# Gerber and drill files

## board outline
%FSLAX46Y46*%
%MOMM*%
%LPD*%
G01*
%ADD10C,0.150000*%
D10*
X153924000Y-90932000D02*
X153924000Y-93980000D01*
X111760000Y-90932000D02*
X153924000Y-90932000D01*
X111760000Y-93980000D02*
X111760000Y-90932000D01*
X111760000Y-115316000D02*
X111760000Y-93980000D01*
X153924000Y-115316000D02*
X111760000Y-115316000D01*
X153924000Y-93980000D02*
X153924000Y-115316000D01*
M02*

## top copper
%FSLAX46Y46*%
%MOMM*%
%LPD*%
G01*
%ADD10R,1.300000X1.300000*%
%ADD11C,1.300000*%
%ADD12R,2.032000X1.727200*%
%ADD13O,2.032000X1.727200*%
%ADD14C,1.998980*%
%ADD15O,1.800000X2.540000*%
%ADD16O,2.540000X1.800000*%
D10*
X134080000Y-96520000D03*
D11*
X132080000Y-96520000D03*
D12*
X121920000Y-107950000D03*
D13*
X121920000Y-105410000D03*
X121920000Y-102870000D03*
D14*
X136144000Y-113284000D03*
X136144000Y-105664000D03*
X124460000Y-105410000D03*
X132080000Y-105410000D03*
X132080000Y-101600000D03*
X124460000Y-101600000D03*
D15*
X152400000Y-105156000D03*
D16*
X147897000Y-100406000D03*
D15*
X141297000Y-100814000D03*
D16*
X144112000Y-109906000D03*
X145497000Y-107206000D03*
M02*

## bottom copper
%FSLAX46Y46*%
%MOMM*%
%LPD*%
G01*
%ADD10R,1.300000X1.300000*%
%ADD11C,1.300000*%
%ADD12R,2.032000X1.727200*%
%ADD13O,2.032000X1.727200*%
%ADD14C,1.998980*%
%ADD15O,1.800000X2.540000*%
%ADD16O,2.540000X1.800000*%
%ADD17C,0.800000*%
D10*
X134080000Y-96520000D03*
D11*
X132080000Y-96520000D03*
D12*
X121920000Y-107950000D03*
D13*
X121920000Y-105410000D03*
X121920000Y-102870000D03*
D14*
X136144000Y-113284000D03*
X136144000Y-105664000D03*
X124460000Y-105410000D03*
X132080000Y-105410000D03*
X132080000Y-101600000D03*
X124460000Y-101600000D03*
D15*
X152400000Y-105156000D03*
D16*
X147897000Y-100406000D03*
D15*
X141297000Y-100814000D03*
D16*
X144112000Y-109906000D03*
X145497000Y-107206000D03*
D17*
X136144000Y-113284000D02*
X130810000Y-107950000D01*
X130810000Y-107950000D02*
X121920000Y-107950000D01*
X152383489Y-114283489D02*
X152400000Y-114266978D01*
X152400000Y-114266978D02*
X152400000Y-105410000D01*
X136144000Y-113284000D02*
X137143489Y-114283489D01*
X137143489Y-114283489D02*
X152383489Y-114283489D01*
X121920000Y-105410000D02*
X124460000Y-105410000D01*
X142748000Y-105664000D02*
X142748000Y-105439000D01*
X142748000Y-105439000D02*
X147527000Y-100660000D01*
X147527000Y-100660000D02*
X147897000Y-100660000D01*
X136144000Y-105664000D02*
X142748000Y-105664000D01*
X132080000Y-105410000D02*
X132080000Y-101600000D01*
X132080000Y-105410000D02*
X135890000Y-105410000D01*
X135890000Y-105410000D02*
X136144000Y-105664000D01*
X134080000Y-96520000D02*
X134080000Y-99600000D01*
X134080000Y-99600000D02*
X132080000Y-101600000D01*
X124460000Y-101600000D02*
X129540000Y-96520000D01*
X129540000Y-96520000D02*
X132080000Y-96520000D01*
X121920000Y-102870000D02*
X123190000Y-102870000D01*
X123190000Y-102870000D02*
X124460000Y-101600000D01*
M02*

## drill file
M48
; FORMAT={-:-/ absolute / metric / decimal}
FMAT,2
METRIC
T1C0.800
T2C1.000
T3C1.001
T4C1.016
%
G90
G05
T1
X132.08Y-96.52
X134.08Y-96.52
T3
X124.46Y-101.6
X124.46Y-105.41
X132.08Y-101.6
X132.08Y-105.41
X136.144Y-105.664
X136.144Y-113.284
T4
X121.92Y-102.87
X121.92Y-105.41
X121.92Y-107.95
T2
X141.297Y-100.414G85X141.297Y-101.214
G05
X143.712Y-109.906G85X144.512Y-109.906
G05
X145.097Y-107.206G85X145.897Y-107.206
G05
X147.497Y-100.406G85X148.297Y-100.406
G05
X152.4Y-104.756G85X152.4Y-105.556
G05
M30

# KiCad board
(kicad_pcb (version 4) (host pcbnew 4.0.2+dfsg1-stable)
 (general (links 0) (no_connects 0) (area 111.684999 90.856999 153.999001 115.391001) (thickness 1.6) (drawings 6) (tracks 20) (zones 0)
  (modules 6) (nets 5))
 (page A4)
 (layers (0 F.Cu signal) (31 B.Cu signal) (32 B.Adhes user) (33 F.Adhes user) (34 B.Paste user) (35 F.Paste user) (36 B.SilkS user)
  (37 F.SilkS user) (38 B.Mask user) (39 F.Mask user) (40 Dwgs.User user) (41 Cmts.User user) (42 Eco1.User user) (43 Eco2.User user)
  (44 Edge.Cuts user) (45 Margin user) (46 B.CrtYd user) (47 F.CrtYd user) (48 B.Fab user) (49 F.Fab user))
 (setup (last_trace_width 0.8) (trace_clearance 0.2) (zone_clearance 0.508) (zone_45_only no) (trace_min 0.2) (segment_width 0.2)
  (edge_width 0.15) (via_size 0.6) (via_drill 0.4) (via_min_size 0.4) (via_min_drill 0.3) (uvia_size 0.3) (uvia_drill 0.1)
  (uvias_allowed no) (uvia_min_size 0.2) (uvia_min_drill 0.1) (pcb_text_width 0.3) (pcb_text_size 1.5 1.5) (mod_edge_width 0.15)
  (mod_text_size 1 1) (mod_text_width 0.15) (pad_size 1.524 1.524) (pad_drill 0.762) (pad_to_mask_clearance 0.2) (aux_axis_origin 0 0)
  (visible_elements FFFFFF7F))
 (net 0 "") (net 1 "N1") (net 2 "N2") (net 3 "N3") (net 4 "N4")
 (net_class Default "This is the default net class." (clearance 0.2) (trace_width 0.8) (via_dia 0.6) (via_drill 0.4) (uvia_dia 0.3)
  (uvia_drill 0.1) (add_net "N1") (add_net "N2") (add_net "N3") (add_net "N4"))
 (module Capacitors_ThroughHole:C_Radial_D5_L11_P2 (layer F.Cu) (at 134.08 96.52 180)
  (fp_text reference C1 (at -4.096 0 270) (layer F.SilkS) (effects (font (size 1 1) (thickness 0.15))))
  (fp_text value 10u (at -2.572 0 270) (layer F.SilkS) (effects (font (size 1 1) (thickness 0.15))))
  (pad 1 thru_hole rect (at 0 0 180) (size 1.3 1.3) (drill 0.8) (layers *.Cu *.Mask F.SilkS) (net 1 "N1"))
  (pad 2 thru_hole circle (at 2 0 180) (size 1.3 1.3) (drill 0.8) (layers *.Cu *.Mask F.SilkS) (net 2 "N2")))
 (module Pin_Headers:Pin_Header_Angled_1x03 (layer F.Cu) (at 121.92 107.95 180)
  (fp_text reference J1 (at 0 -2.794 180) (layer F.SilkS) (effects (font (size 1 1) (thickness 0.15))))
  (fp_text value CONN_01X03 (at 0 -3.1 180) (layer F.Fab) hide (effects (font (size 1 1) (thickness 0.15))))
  (pad 1 thru_hole rect (at 0 0 180) (size 2.032 1.7272) (drill 1.016) (layers *.Cu *.Mask F.SilkS) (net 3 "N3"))
  (pad 2 thru_hole oval (at 0 2.54 180) (size 2.032 1.7272) (drill 1.016) (layers *.Cu *.Mask F.SilkS) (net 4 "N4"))
  (pad 3 thru_hole oval (at 0 5.08 180) (size 2.032 1.7272) (drill 1.016) (layers *.Cu *.Mask F.SilkS) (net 2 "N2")))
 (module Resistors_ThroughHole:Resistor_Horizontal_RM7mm (layer F.Cu) (at 136.144 113.284 90)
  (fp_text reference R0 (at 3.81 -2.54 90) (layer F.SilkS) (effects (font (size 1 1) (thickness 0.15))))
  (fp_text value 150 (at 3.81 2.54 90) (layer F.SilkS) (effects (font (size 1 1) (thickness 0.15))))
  (pad 1 thru_hole circle (at 0 0 90) (size 1.99898 1.99898) (drill 1.00076) (layers *.Cu *.SilkS *.Mask) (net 3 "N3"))
  (pad 2 thru_hole circle (at 7.62 0 90) (size 1.99898 1.99898) (drill 1.00076) (layers *.Cu *.SilkS *.Mask) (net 1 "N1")))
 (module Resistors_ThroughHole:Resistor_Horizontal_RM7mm (layer F.Cu) (at 124.46 105.41)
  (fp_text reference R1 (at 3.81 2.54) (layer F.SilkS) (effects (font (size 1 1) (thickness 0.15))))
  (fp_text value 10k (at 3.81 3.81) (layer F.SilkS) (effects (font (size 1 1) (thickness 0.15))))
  (pad 1 thru_hole circle (at 0 0) (size 1.99898 1.99898) (drill 1.00076) (layers *.Cu *.SilkS *.Mask) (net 4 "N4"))
  (pad 2 thru_hole circle (at 7.62 0) (size 1.99898 1.99898) (drill 1.00076) (layers *.Cu *.SilkS *.Mask) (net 1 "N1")))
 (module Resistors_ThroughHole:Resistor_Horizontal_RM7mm (layer F.Cu) (at 132.08 101.6 180)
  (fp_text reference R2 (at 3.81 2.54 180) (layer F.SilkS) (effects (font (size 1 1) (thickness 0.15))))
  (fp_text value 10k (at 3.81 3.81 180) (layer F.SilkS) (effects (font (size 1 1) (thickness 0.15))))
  (pad 1 thru_hole circle (at 0 0 180) (size 1.99898 1.99898) (drill 1.00076) (layers *.Cu *.SilkS *.Mask) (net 1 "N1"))
  (pad 2 thru_hole circle (at 7.62 0 180) (size 1.99898 1.99898) (drill 1.00076) (layers *.Cu *.SilkS *.Mask) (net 2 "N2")))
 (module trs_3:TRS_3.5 (layer F.Cu) (at 146.812 105.156)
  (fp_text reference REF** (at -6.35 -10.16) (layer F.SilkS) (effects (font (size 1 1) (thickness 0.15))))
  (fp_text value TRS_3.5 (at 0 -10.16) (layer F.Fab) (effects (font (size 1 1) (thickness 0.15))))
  (pad 1 thru_hole oval (at 5.588 0) (size 1.8 2.54) (drill oval 1 1.8) (layers *.Cu *.Mask F.SilkS))
  (pad 3 thru_hole oval (at 1.085 -4.75 90) (size 1.8 2.54) (drill oval 1 1.8) (layers *.Cu *.Mask F.SilkS))
  (pad 5 thru_hole oval (at -5.515 -4.342) (size 1.8 2.54) (drill oval 1 1.8) (layers *.Cu *.Mask F.SilkS))
  (pad 2 thru_hole oval (at -2.7 4.75 90) (size 1.8 2.54) (drill oval 1 1.8) (layers *.Cu *.Mask F.SilkS))
  (pad 4 thru_hole oval (at -1.315 2.05 90) (size 1.8 2.54) (drill oval 1 1.8) (layers *.Cu *.Mask F.SilkS)))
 (gr_line (start 153.924 90.932) (end 153.924 93.98) (layer Edge.Cuts) (width 0.15))
 (gr_line (start 111.76 90.932) (end 153.924 90.932) (layer Edge.Cuts) (width 0.15))
 (gr_line (start 111.76 93.98) (end 111.76 90.932) (layer Edge.Cuts) (width 0.15))
 (gr_line (start 111.76 115.316) (end 111.76 93.98) (layer Edge.Cuts) (width 0.15))
 (gr_line (start 153.924 115.316) (end 111.76 115.316) (layer Edge.Cuts) (width 0.15))
 (gr_line (start 153.924 93.98) (end 153.924 115.316) (layer Edge.Cuts) (width 0.15))
 (segment (start 136.144 113.284) (end 130.81 107.95) (width 0.8) (layer B.Cu) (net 3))
 (segment (start 130.81 107.95) (end 121.92 107.95) (width 0.8) (layer B.Cu) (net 3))
 (segment (start 152.383489 114.283489) (end 152.4 114.266978) (width 0.8) (layer B.Cu) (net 3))
 (segment (start 152.4 114.266978) (end 152.4 105.41) (width 0.8) (layer B.Cu) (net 3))
 (segment (start 136.144 113.284) (end 137.143489 114.283489) (width 0.8) (layer B.Cu) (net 3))
 (segment (start 137.143489 114.283489) (end 152.383489 114.283489) (width 0.8) (layer B.Cu) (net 3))
 (segment (start 121.92 105.41) (end 124.46 105.41) (width 0.8) (layer B.Cu) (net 4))
 (segment (start 142.748 105.664) (end 142.748 105.439) (width 0.8) (layer B.Cu) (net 1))
 (segment (start 142.748 105.439) (end 147.527 100.66) (width 0.8) (layer B.Cu) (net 1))
 (segment (start 147.527 100.66) (end 147.897 100.66) (width 0.8) (layer B.Cu) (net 1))
 (segment (start 136.144 105.664) (end 142.748 105.664) (width 0.8) (layer B.Cu) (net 1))
 (segment (start 132.08 105.41) (end 132.08 101.6) (width 0.8) (layer B.Cu) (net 1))
 (segment (start 132.08 105.41) (end 135.89 105.41) (width 0.8) (layer B.Cu) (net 1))
 (segment (start 135.89 105.41) (end 136.144 105.664) (width 0.8) (layer B.Cu) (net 1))
 (segment (start 134.08 96.52) (end 134.08 99.6) (width 0.8) (layer B.Cu) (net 1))
 (segment (start 134.08 99.6) (end 132.08 101.6) (width 0.8) (layer B.Cu) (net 1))
 (segment (start 124.46 101.6) (end 129.54 96.52) (width 0.8) (layer B.Cu) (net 2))
 (segment (start 129.54 96.52) (end 132.08 96.52) (width 0.8) (layer B.Cu) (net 2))
 (segment (start 121.92 102.87) (end 123.19 102.87) (width 0.8) (layer B.Cu) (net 2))
 (segment (start 123.19 102.87) (end 124.46 101.6) (width 0.8) (layer B.Cu) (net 2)))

